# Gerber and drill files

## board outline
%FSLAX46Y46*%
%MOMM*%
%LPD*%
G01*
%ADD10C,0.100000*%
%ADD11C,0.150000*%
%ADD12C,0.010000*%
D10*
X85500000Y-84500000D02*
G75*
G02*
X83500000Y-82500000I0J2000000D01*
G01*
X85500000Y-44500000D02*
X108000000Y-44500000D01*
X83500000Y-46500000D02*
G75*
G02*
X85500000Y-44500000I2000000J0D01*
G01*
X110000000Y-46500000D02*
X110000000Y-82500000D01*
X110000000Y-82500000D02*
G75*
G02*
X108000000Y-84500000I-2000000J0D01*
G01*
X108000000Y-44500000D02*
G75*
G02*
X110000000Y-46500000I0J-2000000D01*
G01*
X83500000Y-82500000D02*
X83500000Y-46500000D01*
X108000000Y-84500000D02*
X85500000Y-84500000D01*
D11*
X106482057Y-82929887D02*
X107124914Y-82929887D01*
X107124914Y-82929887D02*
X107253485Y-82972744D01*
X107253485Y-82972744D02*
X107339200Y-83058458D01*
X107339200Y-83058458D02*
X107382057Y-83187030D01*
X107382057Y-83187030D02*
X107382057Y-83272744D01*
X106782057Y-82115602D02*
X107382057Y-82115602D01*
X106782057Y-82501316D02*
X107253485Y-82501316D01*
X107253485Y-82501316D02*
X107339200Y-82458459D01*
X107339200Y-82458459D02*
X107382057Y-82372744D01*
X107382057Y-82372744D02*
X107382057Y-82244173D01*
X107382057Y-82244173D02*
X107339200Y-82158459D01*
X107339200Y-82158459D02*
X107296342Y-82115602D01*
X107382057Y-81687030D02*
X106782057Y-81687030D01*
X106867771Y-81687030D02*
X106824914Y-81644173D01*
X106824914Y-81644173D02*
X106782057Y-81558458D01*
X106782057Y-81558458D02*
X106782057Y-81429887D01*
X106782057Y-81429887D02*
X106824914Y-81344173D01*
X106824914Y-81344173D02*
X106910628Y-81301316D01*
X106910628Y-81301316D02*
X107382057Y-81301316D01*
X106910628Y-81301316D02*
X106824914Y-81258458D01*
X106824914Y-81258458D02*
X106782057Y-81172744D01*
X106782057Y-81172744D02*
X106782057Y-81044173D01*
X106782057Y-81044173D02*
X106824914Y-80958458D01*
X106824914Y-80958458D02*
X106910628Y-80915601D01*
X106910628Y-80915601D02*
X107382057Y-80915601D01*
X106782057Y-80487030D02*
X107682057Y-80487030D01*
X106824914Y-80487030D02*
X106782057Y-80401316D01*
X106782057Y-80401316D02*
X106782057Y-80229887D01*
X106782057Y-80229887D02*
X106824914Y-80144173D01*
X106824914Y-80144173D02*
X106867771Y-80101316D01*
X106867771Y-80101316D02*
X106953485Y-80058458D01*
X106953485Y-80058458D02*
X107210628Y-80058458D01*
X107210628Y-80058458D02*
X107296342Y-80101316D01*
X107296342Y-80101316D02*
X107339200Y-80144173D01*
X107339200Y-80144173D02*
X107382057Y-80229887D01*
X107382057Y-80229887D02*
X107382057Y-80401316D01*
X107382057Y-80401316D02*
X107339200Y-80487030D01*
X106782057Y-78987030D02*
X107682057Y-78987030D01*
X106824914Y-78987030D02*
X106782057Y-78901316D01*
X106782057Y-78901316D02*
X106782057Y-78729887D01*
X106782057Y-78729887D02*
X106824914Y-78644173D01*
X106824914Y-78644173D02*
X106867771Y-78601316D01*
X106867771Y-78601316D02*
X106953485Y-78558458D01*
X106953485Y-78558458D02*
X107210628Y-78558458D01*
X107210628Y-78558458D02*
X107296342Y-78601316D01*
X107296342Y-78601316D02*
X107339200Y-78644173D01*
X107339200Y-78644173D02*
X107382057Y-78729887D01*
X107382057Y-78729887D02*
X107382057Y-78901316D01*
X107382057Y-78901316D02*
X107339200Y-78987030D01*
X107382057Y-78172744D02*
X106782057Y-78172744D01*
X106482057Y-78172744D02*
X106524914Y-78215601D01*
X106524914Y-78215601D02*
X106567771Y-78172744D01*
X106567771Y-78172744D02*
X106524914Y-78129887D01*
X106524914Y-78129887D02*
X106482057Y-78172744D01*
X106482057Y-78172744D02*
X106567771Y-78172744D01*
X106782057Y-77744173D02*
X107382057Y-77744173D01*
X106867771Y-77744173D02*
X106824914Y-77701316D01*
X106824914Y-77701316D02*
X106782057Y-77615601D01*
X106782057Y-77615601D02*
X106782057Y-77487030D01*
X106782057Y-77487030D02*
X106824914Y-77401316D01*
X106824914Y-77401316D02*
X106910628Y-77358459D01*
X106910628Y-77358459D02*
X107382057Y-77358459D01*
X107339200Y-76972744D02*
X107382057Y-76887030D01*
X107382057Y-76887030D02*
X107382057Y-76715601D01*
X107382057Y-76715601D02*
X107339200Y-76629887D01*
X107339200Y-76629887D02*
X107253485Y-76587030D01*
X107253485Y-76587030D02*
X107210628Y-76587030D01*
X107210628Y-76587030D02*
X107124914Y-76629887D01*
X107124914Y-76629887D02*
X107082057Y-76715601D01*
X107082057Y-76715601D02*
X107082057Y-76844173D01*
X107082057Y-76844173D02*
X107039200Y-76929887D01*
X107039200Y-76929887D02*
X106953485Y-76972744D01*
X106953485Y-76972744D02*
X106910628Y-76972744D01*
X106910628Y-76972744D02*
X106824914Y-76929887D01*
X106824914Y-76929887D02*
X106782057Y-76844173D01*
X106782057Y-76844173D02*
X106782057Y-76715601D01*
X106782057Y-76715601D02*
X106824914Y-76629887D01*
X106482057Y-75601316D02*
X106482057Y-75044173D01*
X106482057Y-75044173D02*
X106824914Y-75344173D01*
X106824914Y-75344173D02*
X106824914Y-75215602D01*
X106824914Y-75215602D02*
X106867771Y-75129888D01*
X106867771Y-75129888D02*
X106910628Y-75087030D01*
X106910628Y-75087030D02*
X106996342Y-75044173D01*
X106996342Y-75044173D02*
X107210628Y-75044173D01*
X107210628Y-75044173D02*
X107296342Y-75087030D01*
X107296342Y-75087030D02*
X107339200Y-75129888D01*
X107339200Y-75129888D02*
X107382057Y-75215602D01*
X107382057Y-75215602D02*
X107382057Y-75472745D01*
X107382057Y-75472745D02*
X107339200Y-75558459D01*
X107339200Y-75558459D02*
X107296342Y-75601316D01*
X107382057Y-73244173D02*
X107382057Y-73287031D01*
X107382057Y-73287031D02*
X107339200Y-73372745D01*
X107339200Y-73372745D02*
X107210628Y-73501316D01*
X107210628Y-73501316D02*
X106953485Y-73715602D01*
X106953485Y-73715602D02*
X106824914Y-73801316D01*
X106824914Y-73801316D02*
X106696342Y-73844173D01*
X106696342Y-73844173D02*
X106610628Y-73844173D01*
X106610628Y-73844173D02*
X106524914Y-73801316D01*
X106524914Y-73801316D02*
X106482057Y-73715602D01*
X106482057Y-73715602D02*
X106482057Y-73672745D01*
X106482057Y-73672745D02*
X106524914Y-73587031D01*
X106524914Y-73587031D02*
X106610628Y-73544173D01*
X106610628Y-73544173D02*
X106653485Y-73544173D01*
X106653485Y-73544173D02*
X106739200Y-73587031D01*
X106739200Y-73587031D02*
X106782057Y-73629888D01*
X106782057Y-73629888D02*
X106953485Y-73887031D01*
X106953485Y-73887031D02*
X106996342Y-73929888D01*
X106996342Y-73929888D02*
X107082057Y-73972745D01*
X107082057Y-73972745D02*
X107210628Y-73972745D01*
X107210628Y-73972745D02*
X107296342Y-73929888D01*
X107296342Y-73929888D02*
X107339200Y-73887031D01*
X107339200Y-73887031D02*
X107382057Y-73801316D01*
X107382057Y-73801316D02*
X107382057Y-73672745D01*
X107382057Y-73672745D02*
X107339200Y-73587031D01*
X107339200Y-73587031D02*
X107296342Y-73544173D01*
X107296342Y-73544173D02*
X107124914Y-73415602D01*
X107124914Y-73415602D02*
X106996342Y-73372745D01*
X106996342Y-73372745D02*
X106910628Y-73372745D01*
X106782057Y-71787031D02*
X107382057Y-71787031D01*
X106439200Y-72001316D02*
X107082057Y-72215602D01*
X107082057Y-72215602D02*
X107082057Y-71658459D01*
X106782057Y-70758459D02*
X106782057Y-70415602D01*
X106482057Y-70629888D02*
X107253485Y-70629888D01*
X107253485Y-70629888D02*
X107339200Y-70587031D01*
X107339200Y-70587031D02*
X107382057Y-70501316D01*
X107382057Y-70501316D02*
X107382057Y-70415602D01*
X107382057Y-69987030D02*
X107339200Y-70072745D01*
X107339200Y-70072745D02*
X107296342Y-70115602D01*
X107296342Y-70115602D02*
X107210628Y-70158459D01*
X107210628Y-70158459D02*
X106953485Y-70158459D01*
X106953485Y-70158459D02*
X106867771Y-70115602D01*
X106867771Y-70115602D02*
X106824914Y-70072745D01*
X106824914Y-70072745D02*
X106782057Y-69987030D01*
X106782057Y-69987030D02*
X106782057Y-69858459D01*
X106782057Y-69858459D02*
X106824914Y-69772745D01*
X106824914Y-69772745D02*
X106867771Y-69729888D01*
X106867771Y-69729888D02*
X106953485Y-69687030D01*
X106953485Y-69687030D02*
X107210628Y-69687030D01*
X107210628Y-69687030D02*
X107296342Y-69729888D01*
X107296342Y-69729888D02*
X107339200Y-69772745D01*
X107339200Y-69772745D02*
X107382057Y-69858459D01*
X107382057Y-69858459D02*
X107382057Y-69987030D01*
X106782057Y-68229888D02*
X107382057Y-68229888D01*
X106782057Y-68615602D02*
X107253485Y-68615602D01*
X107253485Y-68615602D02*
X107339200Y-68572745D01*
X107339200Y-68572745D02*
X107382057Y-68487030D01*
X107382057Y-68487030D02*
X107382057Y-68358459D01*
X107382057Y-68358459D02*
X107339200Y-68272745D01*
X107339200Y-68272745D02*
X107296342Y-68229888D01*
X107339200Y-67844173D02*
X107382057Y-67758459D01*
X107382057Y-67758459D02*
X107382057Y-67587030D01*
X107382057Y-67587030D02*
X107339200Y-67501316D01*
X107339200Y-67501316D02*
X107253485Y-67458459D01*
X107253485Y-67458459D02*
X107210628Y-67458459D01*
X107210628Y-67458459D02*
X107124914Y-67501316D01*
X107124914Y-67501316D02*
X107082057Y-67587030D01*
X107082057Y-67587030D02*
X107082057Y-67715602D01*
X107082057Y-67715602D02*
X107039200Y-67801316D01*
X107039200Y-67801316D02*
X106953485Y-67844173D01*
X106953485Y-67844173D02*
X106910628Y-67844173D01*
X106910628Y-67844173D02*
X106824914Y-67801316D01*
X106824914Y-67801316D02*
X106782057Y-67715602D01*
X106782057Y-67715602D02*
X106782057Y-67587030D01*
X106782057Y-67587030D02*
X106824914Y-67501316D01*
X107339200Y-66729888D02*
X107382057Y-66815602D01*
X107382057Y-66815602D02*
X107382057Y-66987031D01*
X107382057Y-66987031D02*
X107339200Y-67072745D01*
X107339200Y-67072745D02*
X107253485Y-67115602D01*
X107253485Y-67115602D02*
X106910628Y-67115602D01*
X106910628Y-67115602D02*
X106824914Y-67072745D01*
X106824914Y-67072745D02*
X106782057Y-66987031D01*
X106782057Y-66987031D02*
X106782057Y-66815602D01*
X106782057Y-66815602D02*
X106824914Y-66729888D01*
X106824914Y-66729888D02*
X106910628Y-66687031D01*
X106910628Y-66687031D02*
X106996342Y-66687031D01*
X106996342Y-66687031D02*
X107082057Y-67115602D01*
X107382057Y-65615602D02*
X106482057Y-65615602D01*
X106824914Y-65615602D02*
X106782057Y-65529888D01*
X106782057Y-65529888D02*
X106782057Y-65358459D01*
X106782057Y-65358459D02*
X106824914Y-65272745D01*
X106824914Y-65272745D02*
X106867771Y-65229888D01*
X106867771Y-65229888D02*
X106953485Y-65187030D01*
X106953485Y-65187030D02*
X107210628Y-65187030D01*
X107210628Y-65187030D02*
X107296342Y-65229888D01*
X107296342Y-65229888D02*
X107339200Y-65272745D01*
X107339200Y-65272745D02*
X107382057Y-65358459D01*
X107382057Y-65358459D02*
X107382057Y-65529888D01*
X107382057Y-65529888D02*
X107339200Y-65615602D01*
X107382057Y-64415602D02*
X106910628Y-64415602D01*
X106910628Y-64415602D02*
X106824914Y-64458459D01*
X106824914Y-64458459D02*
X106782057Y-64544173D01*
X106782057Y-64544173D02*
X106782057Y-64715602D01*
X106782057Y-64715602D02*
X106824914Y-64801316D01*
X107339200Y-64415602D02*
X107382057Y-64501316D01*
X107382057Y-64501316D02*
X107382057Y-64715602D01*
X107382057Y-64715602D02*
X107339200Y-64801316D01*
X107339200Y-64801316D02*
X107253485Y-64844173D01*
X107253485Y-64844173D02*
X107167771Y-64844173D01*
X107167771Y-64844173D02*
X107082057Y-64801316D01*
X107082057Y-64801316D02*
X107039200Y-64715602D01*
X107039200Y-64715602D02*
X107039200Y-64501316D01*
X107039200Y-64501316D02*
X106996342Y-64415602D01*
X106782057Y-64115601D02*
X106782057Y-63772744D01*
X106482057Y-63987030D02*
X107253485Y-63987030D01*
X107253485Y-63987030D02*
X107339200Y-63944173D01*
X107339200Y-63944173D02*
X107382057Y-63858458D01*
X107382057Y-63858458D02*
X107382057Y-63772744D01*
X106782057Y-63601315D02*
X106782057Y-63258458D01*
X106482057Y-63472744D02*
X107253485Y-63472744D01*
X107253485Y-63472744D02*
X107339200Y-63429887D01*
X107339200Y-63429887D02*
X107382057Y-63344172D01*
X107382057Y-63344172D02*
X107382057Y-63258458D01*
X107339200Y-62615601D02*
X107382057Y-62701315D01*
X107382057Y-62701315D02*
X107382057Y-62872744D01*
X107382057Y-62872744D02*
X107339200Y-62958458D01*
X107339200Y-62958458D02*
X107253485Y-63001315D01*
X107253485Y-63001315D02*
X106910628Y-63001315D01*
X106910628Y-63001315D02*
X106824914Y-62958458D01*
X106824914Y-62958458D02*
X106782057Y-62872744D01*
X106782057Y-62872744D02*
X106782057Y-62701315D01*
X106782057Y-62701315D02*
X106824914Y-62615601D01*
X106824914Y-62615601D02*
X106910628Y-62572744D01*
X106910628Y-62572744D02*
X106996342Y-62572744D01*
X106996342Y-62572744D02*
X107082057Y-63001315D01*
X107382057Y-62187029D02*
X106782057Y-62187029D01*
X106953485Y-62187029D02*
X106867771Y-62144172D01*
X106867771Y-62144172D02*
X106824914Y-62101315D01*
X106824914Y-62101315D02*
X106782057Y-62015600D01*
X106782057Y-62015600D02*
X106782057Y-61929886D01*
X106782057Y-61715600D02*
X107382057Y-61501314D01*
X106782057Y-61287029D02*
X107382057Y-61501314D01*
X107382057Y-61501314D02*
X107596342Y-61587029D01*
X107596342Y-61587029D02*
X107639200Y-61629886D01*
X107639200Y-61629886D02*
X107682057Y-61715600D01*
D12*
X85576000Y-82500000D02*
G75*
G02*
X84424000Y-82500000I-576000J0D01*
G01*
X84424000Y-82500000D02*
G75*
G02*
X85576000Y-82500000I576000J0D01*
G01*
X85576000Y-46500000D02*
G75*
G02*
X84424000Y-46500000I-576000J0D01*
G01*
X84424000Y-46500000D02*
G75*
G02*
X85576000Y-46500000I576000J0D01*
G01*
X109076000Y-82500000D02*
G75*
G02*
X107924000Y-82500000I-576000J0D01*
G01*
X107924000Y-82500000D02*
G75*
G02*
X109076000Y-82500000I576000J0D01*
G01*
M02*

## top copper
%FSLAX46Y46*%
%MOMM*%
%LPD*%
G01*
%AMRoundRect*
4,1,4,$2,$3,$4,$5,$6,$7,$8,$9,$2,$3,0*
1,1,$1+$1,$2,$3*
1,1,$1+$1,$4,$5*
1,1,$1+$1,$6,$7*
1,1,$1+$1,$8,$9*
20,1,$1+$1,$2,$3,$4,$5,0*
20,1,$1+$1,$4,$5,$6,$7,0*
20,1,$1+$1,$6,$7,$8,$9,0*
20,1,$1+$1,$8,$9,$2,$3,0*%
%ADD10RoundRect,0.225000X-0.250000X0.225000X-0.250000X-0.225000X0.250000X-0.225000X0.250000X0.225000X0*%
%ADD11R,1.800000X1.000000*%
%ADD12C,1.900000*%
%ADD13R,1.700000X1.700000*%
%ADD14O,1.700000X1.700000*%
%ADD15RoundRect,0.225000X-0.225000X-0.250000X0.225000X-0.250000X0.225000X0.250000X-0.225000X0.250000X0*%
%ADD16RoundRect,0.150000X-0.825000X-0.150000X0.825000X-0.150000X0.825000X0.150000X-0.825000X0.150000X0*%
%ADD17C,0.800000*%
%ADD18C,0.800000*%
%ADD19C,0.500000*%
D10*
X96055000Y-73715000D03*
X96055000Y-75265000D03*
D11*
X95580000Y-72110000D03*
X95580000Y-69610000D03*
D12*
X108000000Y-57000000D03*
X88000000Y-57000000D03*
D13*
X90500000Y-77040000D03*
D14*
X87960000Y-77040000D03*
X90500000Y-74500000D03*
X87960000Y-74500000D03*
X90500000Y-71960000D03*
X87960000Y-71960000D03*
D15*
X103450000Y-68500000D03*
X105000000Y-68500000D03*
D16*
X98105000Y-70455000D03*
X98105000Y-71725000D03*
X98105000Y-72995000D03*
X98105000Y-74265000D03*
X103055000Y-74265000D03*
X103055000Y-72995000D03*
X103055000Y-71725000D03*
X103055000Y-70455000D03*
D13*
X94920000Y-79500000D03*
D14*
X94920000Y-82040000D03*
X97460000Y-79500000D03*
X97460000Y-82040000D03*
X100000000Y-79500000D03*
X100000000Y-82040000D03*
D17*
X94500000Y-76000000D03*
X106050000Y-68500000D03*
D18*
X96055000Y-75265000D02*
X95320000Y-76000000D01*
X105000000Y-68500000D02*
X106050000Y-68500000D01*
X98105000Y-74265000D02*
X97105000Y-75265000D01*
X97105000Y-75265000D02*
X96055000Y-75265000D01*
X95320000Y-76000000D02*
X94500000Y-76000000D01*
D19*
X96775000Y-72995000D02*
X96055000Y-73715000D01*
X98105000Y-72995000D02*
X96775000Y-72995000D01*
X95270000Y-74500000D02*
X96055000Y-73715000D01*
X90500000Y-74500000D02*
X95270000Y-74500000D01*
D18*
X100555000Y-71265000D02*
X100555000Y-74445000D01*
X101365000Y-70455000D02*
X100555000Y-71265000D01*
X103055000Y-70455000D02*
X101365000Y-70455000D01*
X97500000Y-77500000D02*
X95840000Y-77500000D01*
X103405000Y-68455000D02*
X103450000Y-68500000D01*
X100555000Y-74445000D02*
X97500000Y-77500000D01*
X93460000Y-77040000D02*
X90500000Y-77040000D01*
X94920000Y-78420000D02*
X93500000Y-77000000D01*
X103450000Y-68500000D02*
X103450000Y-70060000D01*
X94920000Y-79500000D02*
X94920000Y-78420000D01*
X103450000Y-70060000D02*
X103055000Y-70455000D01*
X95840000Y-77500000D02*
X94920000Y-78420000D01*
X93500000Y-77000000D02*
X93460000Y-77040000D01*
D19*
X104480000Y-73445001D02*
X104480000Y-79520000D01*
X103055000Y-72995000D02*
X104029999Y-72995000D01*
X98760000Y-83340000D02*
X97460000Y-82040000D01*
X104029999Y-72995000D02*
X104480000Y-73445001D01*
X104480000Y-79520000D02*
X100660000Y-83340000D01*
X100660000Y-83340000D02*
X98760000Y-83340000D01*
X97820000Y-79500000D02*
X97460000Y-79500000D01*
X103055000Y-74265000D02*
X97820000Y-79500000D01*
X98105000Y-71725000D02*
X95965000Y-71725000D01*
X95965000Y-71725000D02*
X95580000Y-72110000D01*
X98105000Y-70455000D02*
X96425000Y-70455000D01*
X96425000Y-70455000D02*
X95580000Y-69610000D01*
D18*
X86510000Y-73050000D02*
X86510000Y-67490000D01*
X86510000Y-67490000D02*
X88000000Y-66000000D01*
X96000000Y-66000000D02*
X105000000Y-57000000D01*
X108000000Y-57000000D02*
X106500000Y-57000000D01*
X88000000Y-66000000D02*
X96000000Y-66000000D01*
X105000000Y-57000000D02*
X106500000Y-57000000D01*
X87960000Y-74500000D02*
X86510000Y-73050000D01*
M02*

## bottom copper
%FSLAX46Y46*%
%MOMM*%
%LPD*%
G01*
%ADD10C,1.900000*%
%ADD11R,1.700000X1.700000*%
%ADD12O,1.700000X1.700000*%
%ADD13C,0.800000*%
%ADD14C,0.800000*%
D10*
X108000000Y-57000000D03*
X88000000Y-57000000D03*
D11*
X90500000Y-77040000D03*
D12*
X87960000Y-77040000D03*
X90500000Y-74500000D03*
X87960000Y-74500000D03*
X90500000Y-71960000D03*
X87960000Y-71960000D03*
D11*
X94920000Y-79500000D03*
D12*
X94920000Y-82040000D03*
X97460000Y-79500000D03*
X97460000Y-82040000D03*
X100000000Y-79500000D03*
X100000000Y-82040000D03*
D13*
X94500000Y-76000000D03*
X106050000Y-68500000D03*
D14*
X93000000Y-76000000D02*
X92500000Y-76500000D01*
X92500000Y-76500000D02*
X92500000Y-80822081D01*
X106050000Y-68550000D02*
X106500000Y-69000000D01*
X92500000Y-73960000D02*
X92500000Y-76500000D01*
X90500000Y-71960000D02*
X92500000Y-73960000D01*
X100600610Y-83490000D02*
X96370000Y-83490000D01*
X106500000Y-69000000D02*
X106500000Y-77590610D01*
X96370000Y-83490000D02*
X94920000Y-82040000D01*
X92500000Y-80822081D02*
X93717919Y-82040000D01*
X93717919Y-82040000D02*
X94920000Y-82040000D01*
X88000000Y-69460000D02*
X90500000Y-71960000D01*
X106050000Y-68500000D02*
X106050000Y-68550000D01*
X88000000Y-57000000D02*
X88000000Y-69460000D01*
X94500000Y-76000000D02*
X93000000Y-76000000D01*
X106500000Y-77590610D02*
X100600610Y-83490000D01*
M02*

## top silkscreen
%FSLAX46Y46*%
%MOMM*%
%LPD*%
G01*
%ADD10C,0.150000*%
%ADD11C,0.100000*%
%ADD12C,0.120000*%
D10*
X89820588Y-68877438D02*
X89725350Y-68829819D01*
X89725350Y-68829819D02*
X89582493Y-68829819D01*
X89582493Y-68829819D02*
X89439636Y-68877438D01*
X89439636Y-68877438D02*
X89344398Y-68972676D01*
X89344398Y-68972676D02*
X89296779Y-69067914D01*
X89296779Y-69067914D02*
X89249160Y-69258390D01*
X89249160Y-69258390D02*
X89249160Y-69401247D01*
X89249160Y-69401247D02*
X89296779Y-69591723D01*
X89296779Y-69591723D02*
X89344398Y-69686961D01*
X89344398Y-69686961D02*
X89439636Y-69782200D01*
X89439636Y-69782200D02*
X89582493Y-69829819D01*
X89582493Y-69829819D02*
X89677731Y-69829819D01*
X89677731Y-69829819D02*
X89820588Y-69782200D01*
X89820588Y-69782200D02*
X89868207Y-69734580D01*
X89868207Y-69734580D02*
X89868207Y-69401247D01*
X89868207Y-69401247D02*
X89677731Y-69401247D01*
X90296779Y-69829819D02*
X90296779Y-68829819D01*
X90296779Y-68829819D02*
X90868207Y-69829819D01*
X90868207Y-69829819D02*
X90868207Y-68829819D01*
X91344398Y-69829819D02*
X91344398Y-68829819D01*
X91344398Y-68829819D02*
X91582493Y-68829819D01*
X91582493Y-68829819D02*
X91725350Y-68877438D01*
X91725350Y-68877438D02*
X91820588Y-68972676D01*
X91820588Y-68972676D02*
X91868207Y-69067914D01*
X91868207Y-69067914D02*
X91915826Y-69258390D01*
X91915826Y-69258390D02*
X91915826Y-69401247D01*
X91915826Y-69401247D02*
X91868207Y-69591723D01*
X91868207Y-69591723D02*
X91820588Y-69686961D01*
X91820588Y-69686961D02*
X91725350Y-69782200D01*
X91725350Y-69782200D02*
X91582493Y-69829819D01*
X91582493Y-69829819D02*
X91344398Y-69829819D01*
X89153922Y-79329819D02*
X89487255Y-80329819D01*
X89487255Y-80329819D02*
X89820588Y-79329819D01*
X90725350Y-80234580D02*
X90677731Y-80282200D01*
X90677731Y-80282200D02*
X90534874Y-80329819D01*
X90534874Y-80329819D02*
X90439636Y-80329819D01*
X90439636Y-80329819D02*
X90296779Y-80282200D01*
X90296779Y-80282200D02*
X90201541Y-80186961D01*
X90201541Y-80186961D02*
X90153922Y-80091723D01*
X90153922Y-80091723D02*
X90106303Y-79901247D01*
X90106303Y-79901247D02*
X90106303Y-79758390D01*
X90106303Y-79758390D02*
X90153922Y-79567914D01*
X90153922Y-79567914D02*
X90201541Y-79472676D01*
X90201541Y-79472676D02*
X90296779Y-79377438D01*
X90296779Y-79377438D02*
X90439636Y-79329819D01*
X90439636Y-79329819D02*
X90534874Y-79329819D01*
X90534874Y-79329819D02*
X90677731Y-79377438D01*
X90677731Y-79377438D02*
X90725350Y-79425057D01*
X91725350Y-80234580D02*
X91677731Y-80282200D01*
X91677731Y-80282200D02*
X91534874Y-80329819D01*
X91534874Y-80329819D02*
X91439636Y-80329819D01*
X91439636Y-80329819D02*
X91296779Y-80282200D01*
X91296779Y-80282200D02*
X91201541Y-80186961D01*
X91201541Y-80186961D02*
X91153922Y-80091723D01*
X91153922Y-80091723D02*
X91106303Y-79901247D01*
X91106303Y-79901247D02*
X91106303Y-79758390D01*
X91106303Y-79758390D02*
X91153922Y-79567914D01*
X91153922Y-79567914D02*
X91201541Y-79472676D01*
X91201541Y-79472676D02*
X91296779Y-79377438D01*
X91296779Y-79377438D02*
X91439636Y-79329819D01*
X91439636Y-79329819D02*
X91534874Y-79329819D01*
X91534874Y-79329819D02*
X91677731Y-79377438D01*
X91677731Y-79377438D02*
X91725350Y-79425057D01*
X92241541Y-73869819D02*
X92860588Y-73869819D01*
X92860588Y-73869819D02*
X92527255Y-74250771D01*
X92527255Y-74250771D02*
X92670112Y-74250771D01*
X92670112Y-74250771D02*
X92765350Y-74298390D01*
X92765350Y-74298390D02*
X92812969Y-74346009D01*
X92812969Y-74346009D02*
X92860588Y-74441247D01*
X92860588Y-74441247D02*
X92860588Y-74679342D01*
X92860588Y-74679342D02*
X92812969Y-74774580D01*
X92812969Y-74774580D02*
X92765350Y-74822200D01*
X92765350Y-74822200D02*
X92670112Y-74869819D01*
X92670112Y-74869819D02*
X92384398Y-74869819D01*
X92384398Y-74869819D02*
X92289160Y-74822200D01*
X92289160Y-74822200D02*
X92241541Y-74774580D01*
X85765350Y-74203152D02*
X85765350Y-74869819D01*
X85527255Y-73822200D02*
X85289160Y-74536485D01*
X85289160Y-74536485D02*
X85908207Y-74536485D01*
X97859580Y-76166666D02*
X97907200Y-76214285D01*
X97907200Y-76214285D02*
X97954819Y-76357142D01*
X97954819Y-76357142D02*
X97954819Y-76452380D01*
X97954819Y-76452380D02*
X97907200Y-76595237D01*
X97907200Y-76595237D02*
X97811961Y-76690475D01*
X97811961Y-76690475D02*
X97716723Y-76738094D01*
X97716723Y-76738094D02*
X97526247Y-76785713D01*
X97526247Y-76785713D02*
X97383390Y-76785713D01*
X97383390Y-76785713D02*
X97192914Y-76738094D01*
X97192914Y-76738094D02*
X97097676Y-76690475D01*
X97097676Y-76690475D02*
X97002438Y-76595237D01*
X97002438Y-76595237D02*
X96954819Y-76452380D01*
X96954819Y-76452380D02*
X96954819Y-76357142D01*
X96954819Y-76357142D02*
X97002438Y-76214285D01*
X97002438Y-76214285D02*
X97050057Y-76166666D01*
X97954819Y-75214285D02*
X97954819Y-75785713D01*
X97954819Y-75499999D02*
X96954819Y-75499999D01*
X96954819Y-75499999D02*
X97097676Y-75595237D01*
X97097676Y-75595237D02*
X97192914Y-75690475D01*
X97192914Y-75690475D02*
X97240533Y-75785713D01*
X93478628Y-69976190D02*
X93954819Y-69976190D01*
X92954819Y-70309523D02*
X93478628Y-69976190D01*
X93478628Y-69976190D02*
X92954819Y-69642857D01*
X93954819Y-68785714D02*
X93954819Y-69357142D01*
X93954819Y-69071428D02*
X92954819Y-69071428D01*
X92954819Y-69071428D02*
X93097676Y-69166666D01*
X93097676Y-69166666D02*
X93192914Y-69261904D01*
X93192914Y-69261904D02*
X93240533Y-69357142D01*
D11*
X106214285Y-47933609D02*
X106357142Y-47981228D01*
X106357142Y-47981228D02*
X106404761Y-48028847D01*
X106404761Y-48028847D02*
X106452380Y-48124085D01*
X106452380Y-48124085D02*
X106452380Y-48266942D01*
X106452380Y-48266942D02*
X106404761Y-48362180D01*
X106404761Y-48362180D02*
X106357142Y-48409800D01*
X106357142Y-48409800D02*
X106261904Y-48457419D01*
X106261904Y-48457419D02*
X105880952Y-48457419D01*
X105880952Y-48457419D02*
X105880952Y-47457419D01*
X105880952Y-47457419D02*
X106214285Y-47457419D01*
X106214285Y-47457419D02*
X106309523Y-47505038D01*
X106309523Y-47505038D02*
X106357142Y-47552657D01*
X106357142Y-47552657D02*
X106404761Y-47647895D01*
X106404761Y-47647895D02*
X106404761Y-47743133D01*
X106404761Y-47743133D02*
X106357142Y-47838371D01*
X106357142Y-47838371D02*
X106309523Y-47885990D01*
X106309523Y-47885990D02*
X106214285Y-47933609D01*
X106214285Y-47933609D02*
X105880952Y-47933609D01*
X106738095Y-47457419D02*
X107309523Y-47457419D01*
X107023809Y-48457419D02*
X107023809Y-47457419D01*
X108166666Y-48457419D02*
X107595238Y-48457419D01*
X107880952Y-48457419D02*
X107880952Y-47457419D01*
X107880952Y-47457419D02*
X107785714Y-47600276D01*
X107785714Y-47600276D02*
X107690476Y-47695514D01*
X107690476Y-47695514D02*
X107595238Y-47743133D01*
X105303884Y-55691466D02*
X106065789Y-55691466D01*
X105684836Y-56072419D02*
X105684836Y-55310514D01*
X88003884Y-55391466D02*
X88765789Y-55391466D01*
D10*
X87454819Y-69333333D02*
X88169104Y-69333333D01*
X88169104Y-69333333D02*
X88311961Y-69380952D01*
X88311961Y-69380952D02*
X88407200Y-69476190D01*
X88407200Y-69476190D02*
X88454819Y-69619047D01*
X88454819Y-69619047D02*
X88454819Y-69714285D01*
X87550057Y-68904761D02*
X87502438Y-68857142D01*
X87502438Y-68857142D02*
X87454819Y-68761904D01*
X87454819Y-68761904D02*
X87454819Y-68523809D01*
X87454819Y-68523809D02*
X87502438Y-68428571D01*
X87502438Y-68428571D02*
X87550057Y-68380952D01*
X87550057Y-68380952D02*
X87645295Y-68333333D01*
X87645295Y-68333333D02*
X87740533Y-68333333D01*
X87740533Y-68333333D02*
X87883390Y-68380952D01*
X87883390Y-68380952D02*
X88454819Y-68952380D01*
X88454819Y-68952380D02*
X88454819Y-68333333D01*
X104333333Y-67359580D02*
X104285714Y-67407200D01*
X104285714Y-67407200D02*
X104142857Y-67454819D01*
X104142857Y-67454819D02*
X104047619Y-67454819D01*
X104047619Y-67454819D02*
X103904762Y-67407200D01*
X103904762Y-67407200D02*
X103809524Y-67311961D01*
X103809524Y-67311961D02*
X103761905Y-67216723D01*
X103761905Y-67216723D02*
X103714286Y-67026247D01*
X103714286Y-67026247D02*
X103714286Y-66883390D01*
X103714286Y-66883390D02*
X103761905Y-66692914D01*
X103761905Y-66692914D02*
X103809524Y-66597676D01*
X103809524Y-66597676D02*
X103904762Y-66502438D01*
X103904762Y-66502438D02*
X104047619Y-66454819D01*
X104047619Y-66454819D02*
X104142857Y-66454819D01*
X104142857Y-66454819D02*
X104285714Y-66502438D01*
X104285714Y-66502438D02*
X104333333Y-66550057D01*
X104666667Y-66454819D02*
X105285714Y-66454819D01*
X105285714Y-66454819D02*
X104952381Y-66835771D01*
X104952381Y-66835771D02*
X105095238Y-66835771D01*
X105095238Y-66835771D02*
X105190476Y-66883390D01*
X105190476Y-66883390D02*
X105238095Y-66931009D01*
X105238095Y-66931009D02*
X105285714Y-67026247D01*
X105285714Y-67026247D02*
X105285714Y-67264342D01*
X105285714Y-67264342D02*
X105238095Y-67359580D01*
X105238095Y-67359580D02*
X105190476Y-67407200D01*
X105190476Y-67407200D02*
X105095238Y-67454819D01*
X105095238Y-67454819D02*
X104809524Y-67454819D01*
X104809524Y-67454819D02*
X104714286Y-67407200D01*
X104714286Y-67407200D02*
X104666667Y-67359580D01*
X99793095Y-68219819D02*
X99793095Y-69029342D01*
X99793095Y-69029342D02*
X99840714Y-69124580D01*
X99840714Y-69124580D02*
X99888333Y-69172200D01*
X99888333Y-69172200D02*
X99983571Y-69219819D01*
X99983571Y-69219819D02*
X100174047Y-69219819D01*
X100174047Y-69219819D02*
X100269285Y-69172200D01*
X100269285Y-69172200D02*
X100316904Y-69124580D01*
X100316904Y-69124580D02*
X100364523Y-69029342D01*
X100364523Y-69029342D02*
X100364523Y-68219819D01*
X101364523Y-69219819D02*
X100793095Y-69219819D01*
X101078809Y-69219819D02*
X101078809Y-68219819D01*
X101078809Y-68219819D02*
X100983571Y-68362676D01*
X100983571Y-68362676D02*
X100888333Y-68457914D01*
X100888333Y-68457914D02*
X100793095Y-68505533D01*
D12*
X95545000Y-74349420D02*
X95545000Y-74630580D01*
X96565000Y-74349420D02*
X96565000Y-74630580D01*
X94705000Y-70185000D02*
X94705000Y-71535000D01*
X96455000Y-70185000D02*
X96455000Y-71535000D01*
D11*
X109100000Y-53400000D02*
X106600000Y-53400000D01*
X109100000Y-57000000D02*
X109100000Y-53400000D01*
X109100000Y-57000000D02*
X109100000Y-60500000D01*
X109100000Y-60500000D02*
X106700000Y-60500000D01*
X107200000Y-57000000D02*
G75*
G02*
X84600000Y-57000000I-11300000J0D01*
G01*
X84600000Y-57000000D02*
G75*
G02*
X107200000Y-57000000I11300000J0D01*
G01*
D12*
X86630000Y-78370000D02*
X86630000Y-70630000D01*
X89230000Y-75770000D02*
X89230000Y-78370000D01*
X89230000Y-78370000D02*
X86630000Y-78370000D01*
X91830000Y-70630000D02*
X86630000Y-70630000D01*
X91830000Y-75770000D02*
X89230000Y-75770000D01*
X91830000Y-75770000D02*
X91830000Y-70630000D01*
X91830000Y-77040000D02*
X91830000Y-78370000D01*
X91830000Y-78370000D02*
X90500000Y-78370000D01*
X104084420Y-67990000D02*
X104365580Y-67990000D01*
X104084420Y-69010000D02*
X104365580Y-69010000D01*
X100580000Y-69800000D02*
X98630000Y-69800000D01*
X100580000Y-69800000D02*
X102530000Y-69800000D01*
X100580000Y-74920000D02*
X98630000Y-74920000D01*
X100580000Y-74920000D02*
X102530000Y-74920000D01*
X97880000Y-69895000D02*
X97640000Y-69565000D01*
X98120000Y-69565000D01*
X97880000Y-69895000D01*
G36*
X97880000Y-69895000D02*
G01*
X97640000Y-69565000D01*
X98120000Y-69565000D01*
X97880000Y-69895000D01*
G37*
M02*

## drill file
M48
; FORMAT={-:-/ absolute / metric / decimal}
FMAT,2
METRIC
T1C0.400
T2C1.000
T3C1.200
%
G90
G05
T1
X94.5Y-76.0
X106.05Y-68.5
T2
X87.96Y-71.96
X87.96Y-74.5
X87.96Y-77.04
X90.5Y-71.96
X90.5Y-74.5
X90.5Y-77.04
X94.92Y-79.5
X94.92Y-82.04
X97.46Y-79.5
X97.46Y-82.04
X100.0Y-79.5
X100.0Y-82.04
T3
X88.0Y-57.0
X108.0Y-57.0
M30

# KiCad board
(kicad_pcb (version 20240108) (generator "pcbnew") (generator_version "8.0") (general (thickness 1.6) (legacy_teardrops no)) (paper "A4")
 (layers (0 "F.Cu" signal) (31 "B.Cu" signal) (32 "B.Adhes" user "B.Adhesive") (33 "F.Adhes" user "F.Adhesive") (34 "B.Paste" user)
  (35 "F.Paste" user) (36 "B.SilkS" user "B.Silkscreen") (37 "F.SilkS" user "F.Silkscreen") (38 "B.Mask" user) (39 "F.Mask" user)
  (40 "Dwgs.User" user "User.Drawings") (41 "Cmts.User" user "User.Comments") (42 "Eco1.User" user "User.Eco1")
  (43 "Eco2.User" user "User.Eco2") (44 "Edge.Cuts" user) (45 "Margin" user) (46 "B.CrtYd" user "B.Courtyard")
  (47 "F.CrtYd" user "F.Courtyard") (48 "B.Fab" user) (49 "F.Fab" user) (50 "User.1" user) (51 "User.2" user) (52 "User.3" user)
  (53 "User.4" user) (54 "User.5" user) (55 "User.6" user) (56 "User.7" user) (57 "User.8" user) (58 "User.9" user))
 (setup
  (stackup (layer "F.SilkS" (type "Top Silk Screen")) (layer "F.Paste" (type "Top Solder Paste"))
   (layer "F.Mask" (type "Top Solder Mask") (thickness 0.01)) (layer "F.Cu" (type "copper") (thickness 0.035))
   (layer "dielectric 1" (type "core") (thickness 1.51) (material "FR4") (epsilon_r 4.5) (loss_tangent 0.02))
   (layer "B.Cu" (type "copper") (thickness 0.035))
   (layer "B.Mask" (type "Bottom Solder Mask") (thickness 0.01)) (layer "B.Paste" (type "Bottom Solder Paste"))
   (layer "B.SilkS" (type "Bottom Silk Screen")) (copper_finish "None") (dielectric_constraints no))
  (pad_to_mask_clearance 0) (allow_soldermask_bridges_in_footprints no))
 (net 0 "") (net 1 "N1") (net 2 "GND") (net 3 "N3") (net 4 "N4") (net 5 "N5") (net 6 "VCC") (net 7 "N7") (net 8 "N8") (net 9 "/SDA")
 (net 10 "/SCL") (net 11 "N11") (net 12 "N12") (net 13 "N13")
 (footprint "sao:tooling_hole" (layer "F.Cu") (at 85 82.5)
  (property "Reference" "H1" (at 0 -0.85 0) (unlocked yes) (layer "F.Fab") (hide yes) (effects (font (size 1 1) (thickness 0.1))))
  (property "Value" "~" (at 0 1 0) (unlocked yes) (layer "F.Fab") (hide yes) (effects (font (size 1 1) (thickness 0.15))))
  (fp_circle (center 0 0) (end 0.576 0) (stroke (width 0.01) (type default)) (fill none) (layer "Edge.Cuts"))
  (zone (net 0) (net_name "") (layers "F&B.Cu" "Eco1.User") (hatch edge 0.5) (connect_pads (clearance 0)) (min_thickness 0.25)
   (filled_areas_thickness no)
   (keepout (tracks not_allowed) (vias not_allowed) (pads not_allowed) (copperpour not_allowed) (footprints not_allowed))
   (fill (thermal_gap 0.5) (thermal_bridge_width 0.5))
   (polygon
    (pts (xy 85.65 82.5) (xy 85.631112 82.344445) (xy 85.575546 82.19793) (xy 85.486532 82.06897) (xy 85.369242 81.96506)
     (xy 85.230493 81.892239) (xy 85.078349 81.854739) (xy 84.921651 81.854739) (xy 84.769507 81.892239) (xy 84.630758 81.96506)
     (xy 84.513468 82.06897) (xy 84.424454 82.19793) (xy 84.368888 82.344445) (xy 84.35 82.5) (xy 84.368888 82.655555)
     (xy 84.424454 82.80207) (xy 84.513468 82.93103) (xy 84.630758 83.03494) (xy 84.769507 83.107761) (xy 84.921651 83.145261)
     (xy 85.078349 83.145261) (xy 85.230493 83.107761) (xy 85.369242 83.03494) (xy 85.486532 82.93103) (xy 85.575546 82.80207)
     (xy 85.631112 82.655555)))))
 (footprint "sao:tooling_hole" (layer "F.Cu") (at 85 46.5)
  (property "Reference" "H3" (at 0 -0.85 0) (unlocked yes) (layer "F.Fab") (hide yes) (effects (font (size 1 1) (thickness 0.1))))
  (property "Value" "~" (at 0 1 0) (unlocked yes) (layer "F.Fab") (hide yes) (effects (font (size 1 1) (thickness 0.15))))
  (fp_circle (center 0 0) (end 0.576 0) (stroke (width 0.01) (type default)) (fill none) (layer "Edge.Cuts"))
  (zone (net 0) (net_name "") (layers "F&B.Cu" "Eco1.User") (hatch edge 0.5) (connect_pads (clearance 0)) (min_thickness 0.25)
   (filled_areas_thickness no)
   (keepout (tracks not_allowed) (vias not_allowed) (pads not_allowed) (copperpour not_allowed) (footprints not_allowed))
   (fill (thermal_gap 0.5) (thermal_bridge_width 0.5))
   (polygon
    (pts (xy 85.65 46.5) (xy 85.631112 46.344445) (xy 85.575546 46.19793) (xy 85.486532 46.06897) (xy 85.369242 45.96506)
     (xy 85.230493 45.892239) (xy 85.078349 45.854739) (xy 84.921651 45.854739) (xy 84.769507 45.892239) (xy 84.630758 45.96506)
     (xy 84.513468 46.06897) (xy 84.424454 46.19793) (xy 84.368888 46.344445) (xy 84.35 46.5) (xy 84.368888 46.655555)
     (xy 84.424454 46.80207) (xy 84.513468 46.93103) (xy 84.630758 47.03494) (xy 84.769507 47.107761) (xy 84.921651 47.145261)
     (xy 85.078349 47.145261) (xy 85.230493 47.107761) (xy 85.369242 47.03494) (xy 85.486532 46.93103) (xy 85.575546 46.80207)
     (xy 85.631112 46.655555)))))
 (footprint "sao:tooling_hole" (layer "F.Cu") (at 108.5 82.5)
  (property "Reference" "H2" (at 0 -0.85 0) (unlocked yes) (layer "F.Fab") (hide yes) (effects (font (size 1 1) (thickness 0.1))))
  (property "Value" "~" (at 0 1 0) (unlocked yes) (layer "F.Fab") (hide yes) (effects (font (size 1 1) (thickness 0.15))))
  (fp_circle (center 0 0) (end 0.576 0) (stroke (width 0.01) (type default)) (fill none) (layer "Edge.Cuts"))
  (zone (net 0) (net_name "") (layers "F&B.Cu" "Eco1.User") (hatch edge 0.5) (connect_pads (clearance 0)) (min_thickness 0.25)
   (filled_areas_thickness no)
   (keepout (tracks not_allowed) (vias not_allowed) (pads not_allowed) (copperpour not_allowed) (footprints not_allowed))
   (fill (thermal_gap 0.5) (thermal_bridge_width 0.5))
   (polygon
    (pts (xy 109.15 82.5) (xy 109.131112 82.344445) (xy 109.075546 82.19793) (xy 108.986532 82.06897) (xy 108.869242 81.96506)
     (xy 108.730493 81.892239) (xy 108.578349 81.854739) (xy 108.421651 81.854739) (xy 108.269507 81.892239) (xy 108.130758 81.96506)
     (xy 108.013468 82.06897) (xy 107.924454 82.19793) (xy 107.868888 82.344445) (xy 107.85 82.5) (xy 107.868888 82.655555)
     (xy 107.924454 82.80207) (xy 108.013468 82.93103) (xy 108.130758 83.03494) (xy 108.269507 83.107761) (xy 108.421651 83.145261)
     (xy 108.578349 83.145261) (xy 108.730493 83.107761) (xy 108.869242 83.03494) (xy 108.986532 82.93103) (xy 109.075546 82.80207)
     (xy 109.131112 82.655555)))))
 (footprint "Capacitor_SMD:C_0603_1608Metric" (layer "F.Cu") (at 96.055 74.49 -90)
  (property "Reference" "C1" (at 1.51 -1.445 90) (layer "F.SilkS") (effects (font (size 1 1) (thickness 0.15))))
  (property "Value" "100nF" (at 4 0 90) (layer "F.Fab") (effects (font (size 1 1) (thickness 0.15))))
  (fp_line (start -0.14058 0.51) (end 0.14058 0.51) (stroke (width 0.12) (type solid)) (layer "F.SilkS"))
  (fp_line (start -0.14058 -0.51) (end 0.14058 -0.51) (stroke (width 0.12) (type solid)) (layer "F.SilkS"))
  (pad "1" smd roundrect (at -0.775 0 270) (size 0.9 0.95) (layers "F.Cu" "F.Paste" "F.Mask") (roundrect_rratio 0.25) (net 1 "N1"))
  (pad "2" smd roundrect (at 0.775 0 270) (size 0.9 0.95) (layers "F.Cu" "F.Paste" "F.Mask") (roundrect_rratio 0.25) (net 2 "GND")))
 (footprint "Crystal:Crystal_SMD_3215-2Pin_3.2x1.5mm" (layer "F.Cu") (at 95.58 70.86 -90)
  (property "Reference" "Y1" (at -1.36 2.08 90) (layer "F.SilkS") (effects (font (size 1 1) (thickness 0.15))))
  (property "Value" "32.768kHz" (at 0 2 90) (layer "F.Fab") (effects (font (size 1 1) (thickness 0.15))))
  (fp_line (start -0.675 0.875) (end 0.675 0.875) (stroke (width 0.12) (type solid)) (layer "F.SilkS"))
  (fp_line (start -0.675 -0.875) (end 0.675 -0.875) (stroke (width 0.12) (type solid)) (layer "F.SilkS"))
  (pad "1" smd rect (at 1.25 0 270) (size 1 1.8) (layers "F.Cu" "F.Paste" "F.Mask") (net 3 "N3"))
  (pad "2" smd rect (at -1.25 0 270) (size 1 1.8) (layers "F.Cu" "F.Paste" "F.Mask") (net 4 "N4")))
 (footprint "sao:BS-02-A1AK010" (layer "F.Cu") (at 95.9 57)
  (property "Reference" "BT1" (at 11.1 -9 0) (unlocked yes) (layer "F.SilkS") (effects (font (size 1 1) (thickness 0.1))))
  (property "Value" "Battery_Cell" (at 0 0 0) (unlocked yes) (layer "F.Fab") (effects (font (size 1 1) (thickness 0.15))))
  (fp_line (start 13.2 -3.6) (end 10.7 -3.6) (stroke (width 0.1) (type default)) (layer "F.SilkS"))
  (fp_line (start 13.2 0) (end 13.2 -3.6) (stroke (width 0.1) (type default)) (layer "F.SilkS"))
  (fp_line (start 13.2 0) (end 13.2 3.5) (stroke (width 0.1) (type default)) (layer "F.SilkS"))
  (fp_line (start 13.2 3.5) (end 10.8 3.5) (stroke (width 0.1) (type default)) (layer "F.SilkS"))
  (fp_circle (center 0 0) (end 11.3 0) (stroke (width 0.1) (type default)) (fill none) (layer "F.SilkS"))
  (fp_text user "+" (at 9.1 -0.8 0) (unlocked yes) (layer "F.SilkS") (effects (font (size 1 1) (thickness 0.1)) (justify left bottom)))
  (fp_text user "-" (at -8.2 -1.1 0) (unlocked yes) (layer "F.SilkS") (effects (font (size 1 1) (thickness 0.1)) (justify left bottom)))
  (pad "1" thru_hole circle (at 12.1 0) (size 1.9 1.9) (drill 1.2) (layers "*.Cu" "*.Mask") (remove_unused_layers no) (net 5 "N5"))
  (pad "2" thru_hole circle (at -7.9 0) (size 1.9 1.9) (drill 1.2) (layers "*.Cu" "*.Mask") (remove_unused_layers no) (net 2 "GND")))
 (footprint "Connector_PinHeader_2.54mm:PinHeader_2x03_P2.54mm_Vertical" (layer "F.Cu") (at 90.5 77.04 180)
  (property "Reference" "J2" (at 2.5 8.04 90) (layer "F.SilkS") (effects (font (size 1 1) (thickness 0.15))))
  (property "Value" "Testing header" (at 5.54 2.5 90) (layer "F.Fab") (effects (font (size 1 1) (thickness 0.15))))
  (fp_line (start 3.87 -1.33) (end 3.87 6.41) (stroke (width 0.12) (type solid)) (layer "F.SilkS"))
  (fp_line (start 1.27 1.27) (end 1.27 -1.33) (stroke (width 0.12) (type solid)) (layer "F.SilkS"))
  (fp_line (start 1.27 -1.33) (end 3.87 -1.33) (stroke (width 0.12) (type solid)) (layer "F.SilkS"))
  (fp_line (start -1.33 6.41) (end 3.87 6.41) (stroke (width 0.12) (type solid)) (layer "F.SilkS"))
  (fp_line (start -1.33 1.27) (end 1.27 1.27) (stroke (width 0.12) (type solid)) (layer "F.SilkS"))
  (fp_line (start -1.33 1.27) (end -1.33 6.41) (stroke (width 0.12) (type solid)) (layer "F.SilkS"))
  (fp_line (start -1.33 0) (end -1.33 -1.33) (stroke (width 0.12) (type solid)) (layer "F.SilkS"))
  (fp_line (start -1.33 -1.33) (end 0 -1.33) (stroke (width 0.12) (type solid)) (layer "F.SilkS"))
  (pad "1" thru_hole rect (at 0 0 180) (size 1.7 1.7) (drill 1) (layers "*.Cu" "*.Mask") (remove_unused_layers no) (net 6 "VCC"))
  (pad "2" thru_hole oval (at 2.54 0 180) (size 1.7 1.7) (drill 1) (layers "*.Cu" "*.Mask") (remove_unused_layers no) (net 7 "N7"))
  (pad "3" thru_hole oval (at 0 2.54 180) (size 1.7 1.7) (drill 1) (layers "*.Cu" "*.Mask") (remove_unused_layers no) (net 1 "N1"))
  (pad "4" thru_hole oval (at 2.54 2.54 180) (size 1.7 1.7) (drill 1) (layers "*.Cu" "*.Mask") (remove_unused_layers no) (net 5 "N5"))
  (pad "5" thru_hole oval (at 0 5.08 180) (size 1.7 1.7) (drill 1) (layers "*.Cu" "*.Mask") (remove_unused_layers no) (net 2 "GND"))
  (pad "6" thru_hole oval (at 2.54 5.08 180) (size 1.7 1.7) (drill 1) (layers "*.Cu" "*.Mask") (remove_unused_layers no) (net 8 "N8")))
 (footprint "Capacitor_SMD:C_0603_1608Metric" (layer "F.Cu") (at 104.225 68.5)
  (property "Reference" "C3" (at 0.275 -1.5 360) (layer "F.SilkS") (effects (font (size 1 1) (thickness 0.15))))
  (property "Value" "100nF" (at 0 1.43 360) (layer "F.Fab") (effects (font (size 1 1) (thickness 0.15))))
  (fp_line (start -0.14058 -0.51) (end 0.14058 -0.51) (stroke (width 0.12) (type solid)) (layer "F.SilkS"))
  (fp_line (start -0.14058 0.51) (end 0.14058 0.51) (stroke (width 0.12) (type solid)) (layer "F.SilkS"))
  (pad "1" smd roundrect (at -0.775 0) (size 0.9 0.95) (layers "F.Cu" "F.Paste" "F.Mask") (roundrect_rratio 0.25) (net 6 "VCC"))
  (pad "2" smd roundrect (at 0.775 0) (size 0.9 0.95) (layers "F.Cu" "F.Paste" "F.Mask") (roundrect_rratio 0.25) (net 2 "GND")))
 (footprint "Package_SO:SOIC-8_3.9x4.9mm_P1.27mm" (layer "F.Cu") (at 100.58 72.36)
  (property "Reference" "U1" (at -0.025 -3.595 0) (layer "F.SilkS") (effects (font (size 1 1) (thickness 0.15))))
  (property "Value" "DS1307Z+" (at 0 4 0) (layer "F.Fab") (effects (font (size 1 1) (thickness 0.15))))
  (fp_line (start 0 -2.56) (end -1.95 -2.56) (stroke (width 0.12) (type solid)) (layer "F.SilkS"))
  (fp_line (start 0 -2.56) (end 1.95 -2.56) (stroke (width 0.12) (type solid)) (layer "F.SilkS"))
  (fp_line (start 0 2.56) (end -1.95 2.56) (stroke (width 0.12) (type solid)) (layer "F.SilkS"))
  (fp_line (start 0 2.56) (end 1.95 2.56) (stroke (width 0.12) (type solid)) (layer "F.SilkS"))
  (fp_poly
   (pts (xy -2.7 -2.465) (xy -2.94 -2.795) (xy -2.46 -2.795) (xy -2.7 -2.465)) (stroke (width 0.12) (type solid)) (fill solid)
   (layer "F.SilkS"))
  (pad "1" smd roundrect (at -2.475 -1.905) (size 1.95 0.6) (layers "F.Cu" "F.Paste" "F.Mask") (roundrect_rratio 0.25) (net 4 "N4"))
  (pad "2" smd roundrect (at -2.475 -0.635) (size 1.95 0.6) (layers "F.Cu" "F.Paste" "F.Mask") (roundrect_rratio 0.25) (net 3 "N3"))
  (pad "3" smd roundrect (at -2.475 0.635) (size 1.95 0.6) (layers "F.Cu" "F.Paste" "F.Mask") (roundrect_rratio 0.25) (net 1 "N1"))
  (pad "4" smd roundrect (at -2.475 1.905) (size 1.95 0.6) (layers "F.Cu" "F.Paste" "F.Mask") (roundrect_rratio 0.25) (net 2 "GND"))
  (pad "5" smd roundrect (at 2.475 1.905) (size 1.95 0.6) (layers "F.Cu" "F.Paste" "F.Mask") (roundrect_rratio 0.25) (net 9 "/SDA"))
  (pad "6" smd roundrect (at 2.475 0.635) (size 1.95 0.6) (layers "F.Cu" "F.Paste" "F.Mask") (roundrect_rratio 0.25) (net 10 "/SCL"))
  (pad "7" smd roundrect (at 2.475 -0.635) (size 1.95 0.6) (layers "F.Cu" "F.Paste" "F.Mask") (roundrect_rratio 0.25) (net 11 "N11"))
  (pad "8" smd roundrect (at 2.475 -1.905) (size 1.95 0.6) (layers "F.Cu" "F.Paste" "F.Mask") (roundrect_rratio 0.25) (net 6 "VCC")))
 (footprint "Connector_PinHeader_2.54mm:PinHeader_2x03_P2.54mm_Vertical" (layer "B.Cu") (at 94.92 79.5 -90)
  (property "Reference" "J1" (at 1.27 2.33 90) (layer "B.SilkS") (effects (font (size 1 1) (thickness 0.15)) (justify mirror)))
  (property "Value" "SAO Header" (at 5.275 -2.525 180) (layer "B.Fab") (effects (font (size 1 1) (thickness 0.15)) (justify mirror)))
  (pad "1" thru_hole rect (at 0 0 270) (size 1.7 1.7) (drill 1) (layers "*.Cu" "*.Mask") (remove_unused_layers no) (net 6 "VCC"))
  (pad "2" thru_hole oval (at 2.54 0 270) (size 1.7 1.7) (drill 1) (layers "*.Cu" "*.Mask") (remove_unused_layers no) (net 2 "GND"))
  (pad "3" thru_hole oval (at 0 -2.54 270) (size 1.7 1.7) (drill 1) (layers "*.Cu" "*.Mask") (remove_unused_layers no) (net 9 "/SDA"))
  (pad "4" thru_hole oval (at 2.54 -2.54 270) (size 1.7 1.7) (drill 1) (layers "*.Cu" "*.Mask") (remove_unused_layers no) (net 10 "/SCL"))
  (pad "5" thru_hole oval (at 0 -5.08 270) (size 1.7 1.7) (drill 1) (layers "*.Cu" "*.Mask") (remove_unused_layers no) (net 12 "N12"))
  (pad "6" thru_hole oval (at 2.54 -5.08 270) (size 1.7 1.7) (drill 1) (layers "*.Cu" "*.Mask") (remove_unused_layers no) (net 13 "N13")))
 (gr_arc (start 85.5 84.5) (mid 84.085786 83.914214) (end 83.5 82.5) (stroke (width 0.1) (type default)) (layer "Edge.Cuts"))
 (gr_line (start 85.5 44.5) (end 108 44.5) (stroke (width 0.1) (type default)) (layer "Edge.Cuts"))
 (gr_arc (start 83.5 46.5) (mid 84.085786 45.085786) (end 85.5 44.5) (stroke (width 0.1) (type default)) (layer "Edge.Cuts"))
 (gr_line (start 110 46.5) (end 110 82.5) (stroke (width 0.1) (type default)) (layer "Edge.Cuts"))
 (gr_arc (start 110 82.5) (mid 109.414214 83.914214) (end 108 84.5) (stroke (width 0.1) (type default)) (layer "Edge.Cuts"))
 (gr_arc (start 108 44.5) (mid 109.414214 45.085786) (end 110 46.5) (stroke (width 0.1) (type default)) (layer "Edge.Cuts"))
 (gr_line (start 83.5 82.5) (end 83.5 46.5) (stroke (width 0.1) (type default)) (layer "Edge.Cuts"))
 (gr_line (start 108 84.5) (end 85.5 84.5) (stroke (width 0.1) (type default)) (layer "Edge.Cuts"))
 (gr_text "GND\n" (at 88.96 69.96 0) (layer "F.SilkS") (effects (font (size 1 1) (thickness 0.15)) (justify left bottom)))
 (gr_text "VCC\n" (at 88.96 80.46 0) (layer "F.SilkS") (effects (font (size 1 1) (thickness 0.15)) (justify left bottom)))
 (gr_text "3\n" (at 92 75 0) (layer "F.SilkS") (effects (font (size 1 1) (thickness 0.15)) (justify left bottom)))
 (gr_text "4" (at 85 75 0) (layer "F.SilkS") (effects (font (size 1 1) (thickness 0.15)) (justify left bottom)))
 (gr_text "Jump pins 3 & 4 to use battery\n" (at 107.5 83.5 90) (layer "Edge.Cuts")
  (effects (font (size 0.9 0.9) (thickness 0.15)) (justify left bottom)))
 (segment (start 96.055 75.265) (end 95.32 76) (width 0.8) (layer "F.Cu") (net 2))
 (segment (start 105 68.5) (end 106.05 68.5) (width 0.8) (layer "F.Cu") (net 2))
 (segment (start 98.105 74.265) (end 97.105 75.265) (width 0.8) (layer "F.Cu") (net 2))
 (segment (start 97.105 75.265) (end 96.055 75.265) (width 0.8) (layer "F.Cu") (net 2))
 (segment (start 95.32 76) (end 94.5 76) (width 0.8) (layer "F.Cu") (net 2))
 (via (at 94.5 76) (size 0.8) (drill 0.4) (layers "F.Cu" "B.Cu") (free yes) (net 2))
 (via (at 106.05 68.5) (size 0.8) (drill 0.4) (layers "F.Cu" "B.Cu") (free yes) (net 2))
 (segment (start 93 76) (end 92.5 76.5) (width 0.8) (layer "B.Cu") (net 2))
 (segment (start 92.5 76.5) (end 92.5 80.822081) (width 0.8) (layer "B.Cu") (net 2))
 (segment (start 106.05 68.55) (end 106.5 69) (width 0.8) (layer "B.Cu") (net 2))
 (segment (start 92.5 73.96) (end 92.5 76.5) (width 0.8) (layer "B.Cu") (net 2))
 (segment (start 90.5 71.96) (end 92.5 73.96) (width 0.8) (layer "B.Cu") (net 2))
 (segment (start 100.60061 83.49) (end 96.37 83.49) (width 0.8) (layer "B.Cu") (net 2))
 (segment (start 106.5 69) (end 106.5 77.59061) (width 0.8) (layer "B.Cu") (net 2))
 (segment (start 96.37 83.49) (end 94.92 82.04) (width 0.8) (layer "B.Cu") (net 2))
 (segment (start 92.5 80.822081) (end 93.717919 82.04) (width 0.8) (layer "B.Cu") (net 2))
 (segment (start 93.717919 82.04) (end 94.92 82.04) (width 0.8) (layer "B.Cu") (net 2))
 (segment (start 88 69.46) (end 90.5 71.96) (width 0.8) (layer "B.Cu") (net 2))
 (segment (start 106.05 68.5) (end 106.05 68.55) (width 0.8) (layer "B.Cu") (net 2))
 (segment (start 88 57) (end 88 69.46) (width 0.8) (layer "B.Cu") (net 2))
 (segment (start 94.5 76) (end 93 76) (width 0.8) (layer "B.Cu") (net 2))
 (segment (start 106.5 77.59061) (end 100.60061 83.49) (width 0.8) (layer "B.Cu") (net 2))
 (segment (start 96.775 72.995) (end 96.055 73.715) (width 0.5) (layer "F.Cu") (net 1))
 (segment (start 98.105 72.995) (end 96.775 72.995) (width 0.5) (layer "F.Cu") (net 1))
 (segment (start 95.27 74.5) (end 96.055 73.715) (width 0.5) (layer "F.Cu") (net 1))
 (segment (start 90.5 74.5) (end 95.27 74.5) (width 0.5) (layer "F.Cu") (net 1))
 (segment (start 100.555 71.265) (end 100.555 74.445) (width 0.8) (layer "F.Cu") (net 6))
 (segment (start 101.365 70.455) (end 100.555 71.265) (width 0.8) (layer "F.Cu") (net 6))
 (segment (start 103.055 70.455) (end 101.365 70.455) (width 0.8) (layer "F.Cu") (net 6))
 (segment (start 97.5 77.5) (end 95.84 77.5) (width 0.8) (layer "F.Cu") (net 6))
 (segment (start 103.405 68.455) (end 103.45 68.5) (width 0.8) (layer "F.Cu") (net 6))
 (segment (start 100.555 74.445) (end 97.5 77.5) (width 0.8) (layer "F.Cu") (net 6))
 (segment (start 93.46 77.04) (end 90.5 77.04) (width 0.8) (layer "F.Cu") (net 6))
 (segment (start 94.92 78.42) (end 93.5 77) (width 0.8) (layer "F.Cu") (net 6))
 (segment (start 103.45 68.5) (end 103.45 70.06) (width 0.8) (layer "F.Cu") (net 6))
 (segment (start 94.92 79.5) (end 94.92 78.42) (width 0.8) (layer "F.Cu") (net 6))
 (segment (start 103.45 70.06) (end 103.055 70.455) (width 0.8) (layer "F.Cu") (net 6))
 (segment (start 95.84 77.5) (end 94.92 78.42) (width 0.8) (layer "F.Cu") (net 6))
 (segment (start 93.5 77) (end 93.46 77.04) (width 0.8) (layer "F.Cu") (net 6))
 (segment (start 104.48 73.445001) (end 104.48 79.52) (width 0.5) (layer "F.Cu") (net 10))
 (segment (start 103.055 72.995) (end 104.029999 72.995) (width 0.5) (layer "F.Cu") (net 10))
 (segment (start 98.76 83.34) (end 97.46 82.04) (width 0.5) (layer "F.Cu") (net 10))
 (segment (start 104.029999 72.995) (end 104.48 73.445001) (width 0.5) (layer "F.Cu") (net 10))
 (segment (start 104.48 79.52) (end 100.66 83.34) (width 0.5) (layer "F.Cu") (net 10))
 (segment (start 100.66 83.34) (end 98.76 83.34) (width 0.5) (layer "F.Cu") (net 10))
 (segment (start 97.82 79.5) (end 97.46 79.5) (width 0.5) (layer "F.Cu") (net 9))
 (segment (start 103.055 74.265) (end 97.82 79.5) (width 0.5) (layer "F.Cu") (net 9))
 (segment (start 98.105 71.725) (end 95.965 71.725) (width 0.5) (layer "F.Cu") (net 3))
 (segment (start 95.965 71.725) (end 95.58 72.11) (width 0.5) (layer "F.Cu") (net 3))
 (segment (start 98.105 70.455) (end 96.425 70.455) (width 0.5) (layer "F.Cu") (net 4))
 (segment (start 96.425 70.455) (end 95.58 69.61) (width 0.5) (layer "F.Cu") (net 4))
 (segment (start 86.51 73.05) (end 86.51 67.49) (width 0.8) (layer "F.Cu") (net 5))
 (segment (start 86.51 67.49) (end 88 66) (width 0.8) (layer "F.Cu") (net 5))
 (segment (start 96 66) (end 105 57) (width 0.8) (layer "F.Cu") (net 5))
 (segment (start 108 57) (end 106.5 57) (width 0.8) (layer "F.Cu") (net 5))
 (segment (start 88 66) (end 96 66) (width 0.8) (layer "F.Cu") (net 5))
 (segment (start 105 57) (end 106.5 57) (width 0.8) (layer "F.Cu") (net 5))
 (segment (start 87.96 74.5) (end 86.51 73.05) (width 0.8) (layer "F.Cu") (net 5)))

